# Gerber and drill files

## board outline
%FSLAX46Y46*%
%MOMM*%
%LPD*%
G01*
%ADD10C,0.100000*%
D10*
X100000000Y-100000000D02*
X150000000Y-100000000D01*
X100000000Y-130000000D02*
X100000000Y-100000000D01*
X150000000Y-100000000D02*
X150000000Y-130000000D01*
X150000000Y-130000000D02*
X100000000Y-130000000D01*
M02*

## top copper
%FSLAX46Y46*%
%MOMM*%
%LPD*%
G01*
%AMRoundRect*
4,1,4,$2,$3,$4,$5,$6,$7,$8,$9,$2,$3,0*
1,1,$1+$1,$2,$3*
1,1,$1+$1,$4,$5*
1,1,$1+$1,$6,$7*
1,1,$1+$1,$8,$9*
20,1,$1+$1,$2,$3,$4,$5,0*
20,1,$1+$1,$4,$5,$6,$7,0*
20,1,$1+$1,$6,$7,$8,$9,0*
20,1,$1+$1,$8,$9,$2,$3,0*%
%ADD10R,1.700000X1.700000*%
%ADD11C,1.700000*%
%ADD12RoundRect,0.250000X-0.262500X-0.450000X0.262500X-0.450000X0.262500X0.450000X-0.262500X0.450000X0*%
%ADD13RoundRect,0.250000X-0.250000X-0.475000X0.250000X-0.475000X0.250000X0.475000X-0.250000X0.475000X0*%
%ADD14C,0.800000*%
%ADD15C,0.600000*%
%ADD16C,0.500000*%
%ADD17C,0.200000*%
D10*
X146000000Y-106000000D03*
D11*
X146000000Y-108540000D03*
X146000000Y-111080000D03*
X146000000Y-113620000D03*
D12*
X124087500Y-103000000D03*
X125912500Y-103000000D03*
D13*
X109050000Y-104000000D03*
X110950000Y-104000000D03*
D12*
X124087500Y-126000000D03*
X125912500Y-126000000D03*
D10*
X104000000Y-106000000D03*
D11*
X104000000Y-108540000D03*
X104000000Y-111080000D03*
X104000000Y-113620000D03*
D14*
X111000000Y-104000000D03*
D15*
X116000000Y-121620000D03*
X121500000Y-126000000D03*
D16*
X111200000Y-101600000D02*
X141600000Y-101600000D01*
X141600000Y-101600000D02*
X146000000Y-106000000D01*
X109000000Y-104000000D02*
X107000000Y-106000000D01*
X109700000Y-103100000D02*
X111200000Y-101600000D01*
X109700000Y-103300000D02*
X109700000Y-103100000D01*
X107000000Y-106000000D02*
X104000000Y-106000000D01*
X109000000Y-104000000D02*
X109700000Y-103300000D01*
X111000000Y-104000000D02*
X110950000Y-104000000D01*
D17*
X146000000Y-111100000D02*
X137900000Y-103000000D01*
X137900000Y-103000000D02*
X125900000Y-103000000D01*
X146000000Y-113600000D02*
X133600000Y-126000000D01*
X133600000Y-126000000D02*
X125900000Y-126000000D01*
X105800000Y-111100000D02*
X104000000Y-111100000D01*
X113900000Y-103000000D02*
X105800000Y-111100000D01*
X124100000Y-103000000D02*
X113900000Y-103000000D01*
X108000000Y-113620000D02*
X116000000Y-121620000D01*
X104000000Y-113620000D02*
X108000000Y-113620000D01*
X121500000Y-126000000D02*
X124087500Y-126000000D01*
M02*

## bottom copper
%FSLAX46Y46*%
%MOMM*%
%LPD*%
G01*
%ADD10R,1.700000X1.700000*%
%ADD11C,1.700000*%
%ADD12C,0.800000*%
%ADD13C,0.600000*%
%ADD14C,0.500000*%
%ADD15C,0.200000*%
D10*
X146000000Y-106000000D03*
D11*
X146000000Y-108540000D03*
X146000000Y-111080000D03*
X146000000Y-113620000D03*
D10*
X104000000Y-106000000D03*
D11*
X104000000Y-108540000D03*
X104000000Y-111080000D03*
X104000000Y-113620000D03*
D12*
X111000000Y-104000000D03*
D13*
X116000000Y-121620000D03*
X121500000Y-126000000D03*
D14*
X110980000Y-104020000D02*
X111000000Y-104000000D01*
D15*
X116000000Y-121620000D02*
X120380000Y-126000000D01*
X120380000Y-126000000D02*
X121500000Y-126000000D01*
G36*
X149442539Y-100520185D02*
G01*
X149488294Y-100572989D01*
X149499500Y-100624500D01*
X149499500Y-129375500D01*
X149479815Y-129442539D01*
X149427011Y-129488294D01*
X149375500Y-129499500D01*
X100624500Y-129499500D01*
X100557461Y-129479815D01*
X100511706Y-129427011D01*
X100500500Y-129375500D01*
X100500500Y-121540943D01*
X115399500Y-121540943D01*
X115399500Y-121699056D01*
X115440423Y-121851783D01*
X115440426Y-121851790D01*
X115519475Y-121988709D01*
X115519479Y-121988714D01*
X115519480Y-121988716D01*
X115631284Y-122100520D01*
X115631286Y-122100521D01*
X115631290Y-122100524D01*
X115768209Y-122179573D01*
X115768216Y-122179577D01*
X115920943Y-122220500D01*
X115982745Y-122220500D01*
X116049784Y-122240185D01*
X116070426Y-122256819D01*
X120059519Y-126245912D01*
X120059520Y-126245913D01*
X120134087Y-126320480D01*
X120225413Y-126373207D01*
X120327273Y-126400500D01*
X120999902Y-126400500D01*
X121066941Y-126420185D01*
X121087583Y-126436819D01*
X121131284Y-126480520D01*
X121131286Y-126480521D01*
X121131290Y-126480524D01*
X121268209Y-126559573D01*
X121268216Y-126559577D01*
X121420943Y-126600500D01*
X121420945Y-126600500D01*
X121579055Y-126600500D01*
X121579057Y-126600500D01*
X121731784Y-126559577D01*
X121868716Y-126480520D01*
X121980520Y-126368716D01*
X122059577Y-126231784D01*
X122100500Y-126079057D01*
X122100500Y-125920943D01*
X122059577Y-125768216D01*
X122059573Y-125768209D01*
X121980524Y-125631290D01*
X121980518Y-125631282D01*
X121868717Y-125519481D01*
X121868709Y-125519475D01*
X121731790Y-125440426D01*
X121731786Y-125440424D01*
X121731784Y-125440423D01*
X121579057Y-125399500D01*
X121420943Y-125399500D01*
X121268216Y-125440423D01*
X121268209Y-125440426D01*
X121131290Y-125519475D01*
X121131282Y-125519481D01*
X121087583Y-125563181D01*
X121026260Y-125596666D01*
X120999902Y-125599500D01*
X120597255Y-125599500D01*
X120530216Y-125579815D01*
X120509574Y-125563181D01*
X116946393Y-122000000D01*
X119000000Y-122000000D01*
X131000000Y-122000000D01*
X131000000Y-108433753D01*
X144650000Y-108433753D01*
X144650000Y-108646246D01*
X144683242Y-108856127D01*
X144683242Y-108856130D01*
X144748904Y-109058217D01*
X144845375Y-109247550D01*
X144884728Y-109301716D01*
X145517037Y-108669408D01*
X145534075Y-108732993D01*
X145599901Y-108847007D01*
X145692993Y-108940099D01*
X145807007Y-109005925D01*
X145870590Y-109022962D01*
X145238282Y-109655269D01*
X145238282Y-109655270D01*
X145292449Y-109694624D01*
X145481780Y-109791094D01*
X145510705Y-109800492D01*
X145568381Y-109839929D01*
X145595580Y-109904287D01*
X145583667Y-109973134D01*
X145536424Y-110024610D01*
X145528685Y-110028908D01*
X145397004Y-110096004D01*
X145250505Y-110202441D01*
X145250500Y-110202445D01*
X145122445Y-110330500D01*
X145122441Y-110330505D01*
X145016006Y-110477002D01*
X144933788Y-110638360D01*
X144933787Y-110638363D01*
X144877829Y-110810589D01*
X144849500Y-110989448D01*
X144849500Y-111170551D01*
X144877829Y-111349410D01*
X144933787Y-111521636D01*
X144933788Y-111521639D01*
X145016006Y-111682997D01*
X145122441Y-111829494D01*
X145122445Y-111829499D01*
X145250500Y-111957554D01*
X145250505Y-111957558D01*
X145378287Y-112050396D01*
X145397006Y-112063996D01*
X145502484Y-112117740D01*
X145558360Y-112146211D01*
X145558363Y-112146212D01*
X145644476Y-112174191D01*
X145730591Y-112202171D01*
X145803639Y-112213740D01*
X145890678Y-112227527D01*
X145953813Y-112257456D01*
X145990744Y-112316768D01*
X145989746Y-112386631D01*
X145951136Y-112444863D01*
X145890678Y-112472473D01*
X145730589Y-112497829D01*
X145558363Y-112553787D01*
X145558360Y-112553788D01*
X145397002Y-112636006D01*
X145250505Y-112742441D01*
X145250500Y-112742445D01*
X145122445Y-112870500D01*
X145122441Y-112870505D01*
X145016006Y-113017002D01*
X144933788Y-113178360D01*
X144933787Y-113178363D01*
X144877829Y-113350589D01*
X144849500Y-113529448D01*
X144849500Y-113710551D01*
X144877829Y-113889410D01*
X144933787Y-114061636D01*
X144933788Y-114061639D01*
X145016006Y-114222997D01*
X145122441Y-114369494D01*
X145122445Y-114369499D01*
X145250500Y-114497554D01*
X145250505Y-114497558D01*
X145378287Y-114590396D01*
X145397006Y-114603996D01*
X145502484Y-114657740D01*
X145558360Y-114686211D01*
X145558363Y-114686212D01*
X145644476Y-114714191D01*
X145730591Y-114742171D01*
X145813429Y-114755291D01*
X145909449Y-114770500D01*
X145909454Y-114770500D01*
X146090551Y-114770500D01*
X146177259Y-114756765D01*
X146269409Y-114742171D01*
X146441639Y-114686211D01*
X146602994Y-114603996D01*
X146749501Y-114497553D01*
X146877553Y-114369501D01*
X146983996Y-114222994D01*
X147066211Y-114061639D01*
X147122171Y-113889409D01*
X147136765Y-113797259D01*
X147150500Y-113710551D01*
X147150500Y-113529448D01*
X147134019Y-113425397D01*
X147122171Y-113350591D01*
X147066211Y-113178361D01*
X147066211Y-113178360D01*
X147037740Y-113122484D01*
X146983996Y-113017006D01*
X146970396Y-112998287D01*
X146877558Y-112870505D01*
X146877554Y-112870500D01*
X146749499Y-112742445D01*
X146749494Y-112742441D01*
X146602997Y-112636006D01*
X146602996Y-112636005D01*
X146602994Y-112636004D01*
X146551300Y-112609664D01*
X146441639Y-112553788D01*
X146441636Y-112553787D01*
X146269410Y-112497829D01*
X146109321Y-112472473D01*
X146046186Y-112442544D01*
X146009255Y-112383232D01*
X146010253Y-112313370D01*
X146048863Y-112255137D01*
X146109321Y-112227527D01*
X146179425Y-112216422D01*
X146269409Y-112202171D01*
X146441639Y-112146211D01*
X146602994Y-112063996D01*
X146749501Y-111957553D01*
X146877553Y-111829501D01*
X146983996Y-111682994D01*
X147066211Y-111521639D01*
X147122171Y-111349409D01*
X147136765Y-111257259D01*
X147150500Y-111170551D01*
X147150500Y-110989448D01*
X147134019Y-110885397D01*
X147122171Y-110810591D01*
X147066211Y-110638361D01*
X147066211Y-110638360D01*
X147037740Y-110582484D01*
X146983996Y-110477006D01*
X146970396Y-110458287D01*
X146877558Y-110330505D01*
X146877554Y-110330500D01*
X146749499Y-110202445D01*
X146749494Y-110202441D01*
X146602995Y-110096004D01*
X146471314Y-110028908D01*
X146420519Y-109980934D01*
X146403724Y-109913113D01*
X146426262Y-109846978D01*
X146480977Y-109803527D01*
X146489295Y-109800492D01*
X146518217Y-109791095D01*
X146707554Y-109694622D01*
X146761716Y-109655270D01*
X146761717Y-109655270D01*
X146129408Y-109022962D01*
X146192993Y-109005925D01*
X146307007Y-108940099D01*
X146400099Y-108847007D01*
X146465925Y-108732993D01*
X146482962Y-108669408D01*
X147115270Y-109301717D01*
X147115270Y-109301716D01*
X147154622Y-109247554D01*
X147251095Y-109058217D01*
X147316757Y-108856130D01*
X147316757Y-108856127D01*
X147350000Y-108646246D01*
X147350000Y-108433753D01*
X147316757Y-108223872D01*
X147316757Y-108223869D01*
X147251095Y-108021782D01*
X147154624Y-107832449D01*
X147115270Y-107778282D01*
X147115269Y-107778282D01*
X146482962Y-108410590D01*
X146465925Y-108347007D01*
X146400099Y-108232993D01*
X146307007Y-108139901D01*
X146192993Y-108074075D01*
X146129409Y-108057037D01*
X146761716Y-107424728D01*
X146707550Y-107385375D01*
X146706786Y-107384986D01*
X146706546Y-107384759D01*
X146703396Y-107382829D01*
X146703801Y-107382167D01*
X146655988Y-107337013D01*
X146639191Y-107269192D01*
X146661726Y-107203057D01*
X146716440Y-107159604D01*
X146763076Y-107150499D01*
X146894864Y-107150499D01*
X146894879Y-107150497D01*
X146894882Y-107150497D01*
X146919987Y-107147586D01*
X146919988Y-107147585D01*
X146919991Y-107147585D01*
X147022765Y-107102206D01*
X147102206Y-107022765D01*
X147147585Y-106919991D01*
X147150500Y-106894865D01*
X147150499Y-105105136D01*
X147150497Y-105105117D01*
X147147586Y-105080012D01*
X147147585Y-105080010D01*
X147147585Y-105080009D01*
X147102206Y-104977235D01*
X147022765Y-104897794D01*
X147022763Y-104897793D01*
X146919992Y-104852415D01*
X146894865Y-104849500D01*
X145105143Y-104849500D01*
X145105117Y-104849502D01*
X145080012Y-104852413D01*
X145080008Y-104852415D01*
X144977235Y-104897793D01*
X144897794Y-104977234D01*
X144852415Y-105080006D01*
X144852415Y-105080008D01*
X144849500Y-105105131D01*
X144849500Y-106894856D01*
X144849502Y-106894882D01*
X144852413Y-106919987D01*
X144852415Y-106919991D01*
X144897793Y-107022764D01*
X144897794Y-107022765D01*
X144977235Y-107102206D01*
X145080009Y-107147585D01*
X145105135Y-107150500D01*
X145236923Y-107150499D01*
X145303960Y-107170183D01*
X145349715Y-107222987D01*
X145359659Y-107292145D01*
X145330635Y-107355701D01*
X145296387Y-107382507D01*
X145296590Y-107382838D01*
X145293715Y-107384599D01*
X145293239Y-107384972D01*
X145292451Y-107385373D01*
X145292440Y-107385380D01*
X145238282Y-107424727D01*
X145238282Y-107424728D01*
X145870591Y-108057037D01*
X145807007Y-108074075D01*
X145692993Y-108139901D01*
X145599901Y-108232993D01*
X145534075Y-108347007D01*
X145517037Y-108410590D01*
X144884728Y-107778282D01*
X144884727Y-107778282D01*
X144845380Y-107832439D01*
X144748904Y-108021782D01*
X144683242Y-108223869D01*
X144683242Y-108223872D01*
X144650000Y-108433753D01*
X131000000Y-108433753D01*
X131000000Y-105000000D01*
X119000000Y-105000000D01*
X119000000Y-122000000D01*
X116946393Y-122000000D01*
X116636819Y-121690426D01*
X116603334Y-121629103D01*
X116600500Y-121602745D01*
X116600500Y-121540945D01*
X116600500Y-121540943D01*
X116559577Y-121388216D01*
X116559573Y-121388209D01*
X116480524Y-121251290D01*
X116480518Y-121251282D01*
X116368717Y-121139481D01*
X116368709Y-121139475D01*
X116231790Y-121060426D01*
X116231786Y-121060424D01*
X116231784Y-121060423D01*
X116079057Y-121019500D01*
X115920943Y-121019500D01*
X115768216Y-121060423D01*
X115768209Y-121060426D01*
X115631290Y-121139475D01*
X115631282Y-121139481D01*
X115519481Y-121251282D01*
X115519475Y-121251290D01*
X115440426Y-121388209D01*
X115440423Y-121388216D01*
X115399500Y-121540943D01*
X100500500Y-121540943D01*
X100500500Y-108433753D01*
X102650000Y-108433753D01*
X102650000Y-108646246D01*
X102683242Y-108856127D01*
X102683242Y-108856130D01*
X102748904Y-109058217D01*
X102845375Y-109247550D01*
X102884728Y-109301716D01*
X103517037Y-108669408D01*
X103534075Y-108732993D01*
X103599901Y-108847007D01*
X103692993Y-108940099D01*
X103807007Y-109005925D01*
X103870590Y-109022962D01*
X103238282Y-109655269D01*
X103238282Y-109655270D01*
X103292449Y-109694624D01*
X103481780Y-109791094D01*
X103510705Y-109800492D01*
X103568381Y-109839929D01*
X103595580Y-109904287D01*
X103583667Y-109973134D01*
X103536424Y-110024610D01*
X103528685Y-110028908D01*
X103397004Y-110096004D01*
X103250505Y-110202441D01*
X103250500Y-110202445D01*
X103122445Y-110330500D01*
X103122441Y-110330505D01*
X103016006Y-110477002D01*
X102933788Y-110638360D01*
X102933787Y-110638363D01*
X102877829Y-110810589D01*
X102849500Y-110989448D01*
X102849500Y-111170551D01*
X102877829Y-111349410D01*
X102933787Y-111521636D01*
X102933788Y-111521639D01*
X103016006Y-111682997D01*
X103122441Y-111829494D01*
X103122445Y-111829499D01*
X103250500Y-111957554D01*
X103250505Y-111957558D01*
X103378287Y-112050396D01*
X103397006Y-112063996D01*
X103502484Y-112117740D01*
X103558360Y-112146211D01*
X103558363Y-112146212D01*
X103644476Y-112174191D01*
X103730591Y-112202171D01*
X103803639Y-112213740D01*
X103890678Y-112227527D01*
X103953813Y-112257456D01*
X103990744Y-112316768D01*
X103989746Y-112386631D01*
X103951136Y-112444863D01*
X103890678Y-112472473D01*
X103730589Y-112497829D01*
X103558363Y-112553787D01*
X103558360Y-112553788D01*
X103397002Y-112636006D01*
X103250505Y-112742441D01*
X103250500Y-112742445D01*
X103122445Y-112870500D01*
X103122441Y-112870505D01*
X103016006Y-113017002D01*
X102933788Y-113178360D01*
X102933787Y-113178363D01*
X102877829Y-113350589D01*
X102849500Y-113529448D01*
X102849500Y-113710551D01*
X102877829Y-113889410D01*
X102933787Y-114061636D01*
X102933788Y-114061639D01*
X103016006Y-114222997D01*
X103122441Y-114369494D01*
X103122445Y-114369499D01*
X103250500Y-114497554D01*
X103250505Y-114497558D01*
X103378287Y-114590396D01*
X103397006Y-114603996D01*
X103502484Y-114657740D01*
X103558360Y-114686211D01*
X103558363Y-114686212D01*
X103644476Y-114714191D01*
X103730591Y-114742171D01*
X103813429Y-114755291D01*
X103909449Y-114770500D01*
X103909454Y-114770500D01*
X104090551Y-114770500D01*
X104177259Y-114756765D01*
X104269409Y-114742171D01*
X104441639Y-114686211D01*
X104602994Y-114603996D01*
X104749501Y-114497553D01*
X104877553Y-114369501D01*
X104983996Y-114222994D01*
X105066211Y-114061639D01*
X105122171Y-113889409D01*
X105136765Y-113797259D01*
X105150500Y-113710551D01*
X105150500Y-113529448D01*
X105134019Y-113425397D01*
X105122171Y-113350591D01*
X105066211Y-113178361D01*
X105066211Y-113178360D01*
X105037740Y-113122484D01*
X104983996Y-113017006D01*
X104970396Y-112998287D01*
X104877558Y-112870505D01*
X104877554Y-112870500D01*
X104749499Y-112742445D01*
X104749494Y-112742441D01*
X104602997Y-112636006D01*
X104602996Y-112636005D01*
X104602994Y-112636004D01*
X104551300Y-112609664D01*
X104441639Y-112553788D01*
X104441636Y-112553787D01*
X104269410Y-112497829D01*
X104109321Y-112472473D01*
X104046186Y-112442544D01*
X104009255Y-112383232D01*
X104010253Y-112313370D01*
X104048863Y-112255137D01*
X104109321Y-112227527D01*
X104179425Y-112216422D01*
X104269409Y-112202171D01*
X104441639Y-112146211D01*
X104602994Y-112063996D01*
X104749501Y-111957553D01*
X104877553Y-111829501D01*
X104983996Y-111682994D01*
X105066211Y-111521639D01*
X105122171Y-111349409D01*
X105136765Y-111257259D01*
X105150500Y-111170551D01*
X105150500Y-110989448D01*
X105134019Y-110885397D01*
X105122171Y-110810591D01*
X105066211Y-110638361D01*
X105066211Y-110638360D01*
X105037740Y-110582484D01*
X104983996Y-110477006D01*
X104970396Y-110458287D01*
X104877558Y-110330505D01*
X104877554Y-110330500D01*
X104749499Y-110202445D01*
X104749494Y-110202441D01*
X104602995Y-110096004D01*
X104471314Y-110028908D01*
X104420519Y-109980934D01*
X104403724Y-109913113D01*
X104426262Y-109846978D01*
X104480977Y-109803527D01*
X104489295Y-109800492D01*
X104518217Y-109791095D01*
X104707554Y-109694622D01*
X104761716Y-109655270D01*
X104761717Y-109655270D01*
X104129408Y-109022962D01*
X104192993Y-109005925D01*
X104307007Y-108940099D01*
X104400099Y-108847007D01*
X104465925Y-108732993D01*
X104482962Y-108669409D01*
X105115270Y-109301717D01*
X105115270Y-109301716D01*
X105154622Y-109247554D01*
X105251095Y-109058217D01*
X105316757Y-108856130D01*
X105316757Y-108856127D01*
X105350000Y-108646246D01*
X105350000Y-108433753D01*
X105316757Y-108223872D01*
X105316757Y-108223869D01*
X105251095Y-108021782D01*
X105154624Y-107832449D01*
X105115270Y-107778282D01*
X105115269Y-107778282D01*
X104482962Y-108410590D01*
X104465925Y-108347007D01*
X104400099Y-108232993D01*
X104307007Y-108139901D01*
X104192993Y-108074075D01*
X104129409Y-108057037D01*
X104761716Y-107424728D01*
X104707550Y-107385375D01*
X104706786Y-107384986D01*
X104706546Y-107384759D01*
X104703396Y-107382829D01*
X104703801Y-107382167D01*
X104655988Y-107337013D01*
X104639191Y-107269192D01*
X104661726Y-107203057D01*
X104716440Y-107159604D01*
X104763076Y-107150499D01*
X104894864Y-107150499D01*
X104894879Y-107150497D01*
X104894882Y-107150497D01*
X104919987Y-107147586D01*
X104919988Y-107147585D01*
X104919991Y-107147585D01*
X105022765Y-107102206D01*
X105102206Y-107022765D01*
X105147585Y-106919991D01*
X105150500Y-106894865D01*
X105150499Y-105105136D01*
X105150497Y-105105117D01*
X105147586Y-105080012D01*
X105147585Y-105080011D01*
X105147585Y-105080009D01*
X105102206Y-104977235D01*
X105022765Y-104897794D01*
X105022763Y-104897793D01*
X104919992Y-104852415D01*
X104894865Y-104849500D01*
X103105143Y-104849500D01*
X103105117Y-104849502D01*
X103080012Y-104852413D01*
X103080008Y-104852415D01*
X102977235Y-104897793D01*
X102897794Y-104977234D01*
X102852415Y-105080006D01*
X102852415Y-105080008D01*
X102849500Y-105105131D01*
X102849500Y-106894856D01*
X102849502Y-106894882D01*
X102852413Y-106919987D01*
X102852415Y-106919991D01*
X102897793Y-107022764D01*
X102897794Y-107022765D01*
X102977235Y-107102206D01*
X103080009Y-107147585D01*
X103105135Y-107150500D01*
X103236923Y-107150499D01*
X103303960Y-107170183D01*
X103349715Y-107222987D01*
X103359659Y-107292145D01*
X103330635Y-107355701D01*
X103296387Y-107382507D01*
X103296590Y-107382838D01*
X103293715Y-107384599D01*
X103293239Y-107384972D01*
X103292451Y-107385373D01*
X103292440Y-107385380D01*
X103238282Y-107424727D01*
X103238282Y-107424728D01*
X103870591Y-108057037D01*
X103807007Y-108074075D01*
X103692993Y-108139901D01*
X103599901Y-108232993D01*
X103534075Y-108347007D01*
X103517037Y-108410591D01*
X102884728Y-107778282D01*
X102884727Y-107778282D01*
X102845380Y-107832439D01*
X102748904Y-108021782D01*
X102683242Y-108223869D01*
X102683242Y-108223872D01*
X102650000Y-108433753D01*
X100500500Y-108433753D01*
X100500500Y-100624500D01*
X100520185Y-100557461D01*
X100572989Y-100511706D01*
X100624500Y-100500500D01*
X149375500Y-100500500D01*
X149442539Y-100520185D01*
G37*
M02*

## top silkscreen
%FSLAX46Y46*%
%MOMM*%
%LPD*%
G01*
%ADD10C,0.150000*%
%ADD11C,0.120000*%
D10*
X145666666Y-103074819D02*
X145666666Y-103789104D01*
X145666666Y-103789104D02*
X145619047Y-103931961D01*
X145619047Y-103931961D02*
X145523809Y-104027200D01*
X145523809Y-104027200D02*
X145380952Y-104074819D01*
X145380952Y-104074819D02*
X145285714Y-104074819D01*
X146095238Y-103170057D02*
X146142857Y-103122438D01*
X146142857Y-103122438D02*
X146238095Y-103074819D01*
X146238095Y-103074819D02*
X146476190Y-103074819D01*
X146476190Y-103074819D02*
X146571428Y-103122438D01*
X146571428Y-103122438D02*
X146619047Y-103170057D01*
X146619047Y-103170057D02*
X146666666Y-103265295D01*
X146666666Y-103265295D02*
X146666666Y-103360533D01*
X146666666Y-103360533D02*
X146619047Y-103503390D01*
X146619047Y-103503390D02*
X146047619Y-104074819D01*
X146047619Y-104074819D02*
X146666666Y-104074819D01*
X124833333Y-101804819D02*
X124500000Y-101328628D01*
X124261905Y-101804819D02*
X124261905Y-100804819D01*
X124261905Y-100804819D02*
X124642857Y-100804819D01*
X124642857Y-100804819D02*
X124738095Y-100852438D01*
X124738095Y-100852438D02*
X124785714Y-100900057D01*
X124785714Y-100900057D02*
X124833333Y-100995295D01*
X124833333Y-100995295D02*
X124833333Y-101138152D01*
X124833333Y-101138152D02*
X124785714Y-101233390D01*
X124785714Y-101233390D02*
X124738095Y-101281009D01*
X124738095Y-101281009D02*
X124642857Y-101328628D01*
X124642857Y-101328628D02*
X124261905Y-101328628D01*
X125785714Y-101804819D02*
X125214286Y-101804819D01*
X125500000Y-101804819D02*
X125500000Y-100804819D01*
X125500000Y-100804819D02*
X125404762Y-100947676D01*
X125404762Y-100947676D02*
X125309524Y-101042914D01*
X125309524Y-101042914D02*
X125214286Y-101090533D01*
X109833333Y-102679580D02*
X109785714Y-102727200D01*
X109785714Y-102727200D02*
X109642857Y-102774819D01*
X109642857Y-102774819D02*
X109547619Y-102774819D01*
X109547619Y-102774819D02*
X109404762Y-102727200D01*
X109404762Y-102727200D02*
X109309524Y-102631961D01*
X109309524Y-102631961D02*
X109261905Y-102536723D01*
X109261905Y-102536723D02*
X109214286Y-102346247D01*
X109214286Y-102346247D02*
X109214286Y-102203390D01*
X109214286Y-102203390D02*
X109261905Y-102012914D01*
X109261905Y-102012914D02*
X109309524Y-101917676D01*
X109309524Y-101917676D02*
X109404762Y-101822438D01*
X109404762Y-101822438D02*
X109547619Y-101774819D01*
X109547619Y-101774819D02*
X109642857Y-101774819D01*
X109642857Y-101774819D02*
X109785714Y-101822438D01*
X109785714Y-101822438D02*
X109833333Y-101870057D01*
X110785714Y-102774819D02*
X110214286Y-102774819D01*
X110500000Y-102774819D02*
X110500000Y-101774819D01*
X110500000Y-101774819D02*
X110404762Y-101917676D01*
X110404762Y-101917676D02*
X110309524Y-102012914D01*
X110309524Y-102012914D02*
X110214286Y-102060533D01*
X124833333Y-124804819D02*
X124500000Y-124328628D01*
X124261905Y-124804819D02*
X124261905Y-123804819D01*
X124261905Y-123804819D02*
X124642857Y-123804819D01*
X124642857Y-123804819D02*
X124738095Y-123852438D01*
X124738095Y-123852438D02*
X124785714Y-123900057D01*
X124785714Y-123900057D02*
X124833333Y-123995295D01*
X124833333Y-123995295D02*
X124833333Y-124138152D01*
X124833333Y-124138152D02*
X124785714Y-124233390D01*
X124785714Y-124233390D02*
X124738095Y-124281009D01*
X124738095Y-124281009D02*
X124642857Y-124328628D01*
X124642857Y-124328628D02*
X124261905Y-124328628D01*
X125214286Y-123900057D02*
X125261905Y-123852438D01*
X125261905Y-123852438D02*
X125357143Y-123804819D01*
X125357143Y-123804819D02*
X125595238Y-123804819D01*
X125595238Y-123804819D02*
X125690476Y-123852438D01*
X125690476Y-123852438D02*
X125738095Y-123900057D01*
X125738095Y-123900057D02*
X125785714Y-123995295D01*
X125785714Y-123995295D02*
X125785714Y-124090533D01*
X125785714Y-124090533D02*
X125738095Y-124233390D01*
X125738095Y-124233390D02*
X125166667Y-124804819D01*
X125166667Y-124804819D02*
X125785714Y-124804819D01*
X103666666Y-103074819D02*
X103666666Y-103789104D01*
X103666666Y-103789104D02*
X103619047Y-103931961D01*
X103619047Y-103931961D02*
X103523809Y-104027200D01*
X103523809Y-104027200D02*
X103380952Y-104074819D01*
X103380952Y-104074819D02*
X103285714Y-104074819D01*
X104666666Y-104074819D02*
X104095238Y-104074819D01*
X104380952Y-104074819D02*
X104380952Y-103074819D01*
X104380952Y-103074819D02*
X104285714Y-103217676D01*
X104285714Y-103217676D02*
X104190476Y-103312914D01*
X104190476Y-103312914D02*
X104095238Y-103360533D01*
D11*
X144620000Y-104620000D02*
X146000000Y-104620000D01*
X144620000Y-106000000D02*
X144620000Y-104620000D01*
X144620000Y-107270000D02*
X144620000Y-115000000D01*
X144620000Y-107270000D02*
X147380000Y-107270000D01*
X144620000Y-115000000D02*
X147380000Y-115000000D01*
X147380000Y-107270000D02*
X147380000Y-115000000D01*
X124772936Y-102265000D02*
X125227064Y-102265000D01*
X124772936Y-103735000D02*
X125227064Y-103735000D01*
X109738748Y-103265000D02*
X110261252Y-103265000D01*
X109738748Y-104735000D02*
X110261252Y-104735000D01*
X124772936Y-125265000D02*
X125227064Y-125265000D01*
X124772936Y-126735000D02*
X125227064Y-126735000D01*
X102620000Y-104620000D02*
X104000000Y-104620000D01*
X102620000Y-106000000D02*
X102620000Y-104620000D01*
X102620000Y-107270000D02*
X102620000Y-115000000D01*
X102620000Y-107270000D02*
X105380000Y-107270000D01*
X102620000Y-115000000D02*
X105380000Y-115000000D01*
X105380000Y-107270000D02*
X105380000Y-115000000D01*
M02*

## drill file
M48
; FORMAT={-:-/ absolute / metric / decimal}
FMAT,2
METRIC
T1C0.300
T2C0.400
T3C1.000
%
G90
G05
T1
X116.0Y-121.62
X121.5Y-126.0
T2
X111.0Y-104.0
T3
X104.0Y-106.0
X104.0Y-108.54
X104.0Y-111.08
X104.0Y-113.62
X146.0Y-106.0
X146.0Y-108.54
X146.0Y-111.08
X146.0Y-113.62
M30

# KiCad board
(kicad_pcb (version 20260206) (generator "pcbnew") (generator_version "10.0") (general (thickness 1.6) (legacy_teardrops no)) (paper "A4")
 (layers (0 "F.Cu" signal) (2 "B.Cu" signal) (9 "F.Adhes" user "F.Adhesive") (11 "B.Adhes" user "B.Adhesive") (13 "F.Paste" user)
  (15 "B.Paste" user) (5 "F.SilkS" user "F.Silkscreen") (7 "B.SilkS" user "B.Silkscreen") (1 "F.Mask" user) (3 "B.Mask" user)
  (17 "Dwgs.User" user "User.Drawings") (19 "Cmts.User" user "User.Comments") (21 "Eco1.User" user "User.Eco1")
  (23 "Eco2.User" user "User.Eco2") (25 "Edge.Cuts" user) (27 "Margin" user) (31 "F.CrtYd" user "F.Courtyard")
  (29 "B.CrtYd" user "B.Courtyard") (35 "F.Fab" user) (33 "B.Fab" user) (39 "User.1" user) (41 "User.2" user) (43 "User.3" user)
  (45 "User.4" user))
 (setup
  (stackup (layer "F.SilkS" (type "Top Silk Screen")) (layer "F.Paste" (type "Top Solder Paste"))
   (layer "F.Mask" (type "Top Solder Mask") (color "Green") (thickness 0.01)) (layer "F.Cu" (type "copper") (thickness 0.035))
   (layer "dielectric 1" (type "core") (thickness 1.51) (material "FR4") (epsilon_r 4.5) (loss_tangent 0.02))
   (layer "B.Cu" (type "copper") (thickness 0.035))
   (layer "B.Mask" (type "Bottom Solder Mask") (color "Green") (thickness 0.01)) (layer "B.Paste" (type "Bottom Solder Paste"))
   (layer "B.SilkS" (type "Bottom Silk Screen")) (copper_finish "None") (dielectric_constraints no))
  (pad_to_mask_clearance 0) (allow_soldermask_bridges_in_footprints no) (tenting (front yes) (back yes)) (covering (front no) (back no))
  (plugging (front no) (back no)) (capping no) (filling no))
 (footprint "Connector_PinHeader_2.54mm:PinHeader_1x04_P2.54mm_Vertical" (layer "F.Cu") (at 146 106)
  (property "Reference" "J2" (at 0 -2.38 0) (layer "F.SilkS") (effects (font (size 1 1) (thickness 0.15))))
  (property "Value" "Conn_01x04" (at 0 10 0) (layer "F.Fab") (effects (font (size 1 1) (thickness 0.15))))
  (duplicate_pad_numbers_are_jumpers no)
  (fp_line (start -1.38 -1.38) (end 0 -1.38) (stroke (width 0.12) (type solid)) (layer "F.SilkS"))
  (fp_line (start -1.38 0) (end -1.38 -1.38) (stroke (width 0.12) (type solid)) (layer "F.SilkS"))
  (fp_line (start -1.38 1.27) (end -1.38 9) (stroke (width 0.12) (type solid)) (layer "F.SilkS"))
  (fp_line (start -1.38 1.27) (end 1.38 1.27) (stroke (width 0.12) (type solid)) (layer "F.SilkS"))
  (fp_line (start -1.38 9) (end 1.38 9) (stroke (width 0.12) (type solid)) (layer "F.SilkS"))
  (fp_line (start 1.38 1.27) (end 1.38 9) (stroke (width 0.12) (type solid)) (layer "F.SilkS"))
  (pad "1" thru_hole rect (at 0 0) (size 1.7 1.7) (drill 1) (layers "*.Cu" "*.Mask") (remove_unused_layers no) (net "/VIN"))
  (pad "2" thru_hole circle (at 0 2.54) (size 1.7 1.7) (drill 1) (layers "*.Cu" "*.Mask") (remove_unused_layers no) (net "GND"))
  (pad "3" thru_hole circle (at 0 5.08) (size 1.7 1.7) (drill 1) (layers "*.Cu" "*.Mask") (remove_unused_layers no) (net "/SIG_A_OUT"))
  (pad "4" thru_hole circle (at 0 7.62) (size 1.7 1.7) (drill 1) (layers "*.Cu" "*.Mask") (remove_unused_layers no) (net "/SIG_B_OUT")))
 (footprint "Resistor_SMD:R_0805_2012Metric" (layer "F.Cu") (at 125 103)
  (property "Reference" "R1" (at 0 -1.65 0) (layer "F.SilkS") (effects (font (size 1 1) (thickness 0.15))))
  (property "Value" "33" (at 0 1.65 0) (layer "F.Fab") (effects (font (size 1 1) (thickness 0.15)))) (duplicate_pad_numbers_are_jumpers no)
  (fp_line (start -0.227064 -0.735) (end 0.227064 -0.735) (stroke (width 0.12) (type solid)) (layer "F.SilkS"))
  (fp_line (start -0.227064 0.735) (end 0.227064 0.735) (stroke (width 0.12) (type solid)) (layer "F.SilkS"))
  (pad "1" smd roundrect (at -0.9125 0) (size 1.025 1.4) (layers "F.Cu" "F.Mask" "F.Paste") (roundrect_rratio 0.243902) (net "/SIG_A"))
  (pad "2" smd roundrect (at 0.9125 0) (size 1.025 1.4) (layers "F.Cu" "F.Mask" "F.Paste") (roundrect_rratio 0.243902) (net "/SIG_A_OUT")))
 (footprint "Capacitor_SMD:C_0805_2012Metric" (layer "F.Cu") (at 110 104)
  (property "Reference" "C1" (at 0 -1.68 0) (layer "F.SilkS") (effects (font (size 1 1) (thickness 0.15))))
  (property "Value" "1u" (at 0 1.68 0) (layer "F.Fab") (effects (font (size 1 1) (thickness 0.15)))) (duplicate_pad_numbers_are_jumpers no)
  (fp_line (start -0.261252 -0.735) (end 0.261252 -0.735) (stroke (width 0.12) (type solid)) (layer "F.SilkS"))
  (fp_line (start -0.261252 0.735) (end 0.261252 0.735) (stroke (width 0.12) (type solid)) (layer "F.SilkS"))
  (pad "1" smd roundrect (at -0.95 0) (size 1 1.45) (layers "F.Cu" "F.Mask" "F.Paste") (roundrect_rratio 0.25) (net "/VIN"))
  (pad "2" smd roundrect (at 0.95 0) (size 1 1.45) (layers "F.Cu" "F.Mask" "F.Paste") (roundrect_rratio 0.25) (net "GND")))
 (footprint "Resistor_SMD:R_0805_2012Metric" (layer "F.Cu") (at 125 126)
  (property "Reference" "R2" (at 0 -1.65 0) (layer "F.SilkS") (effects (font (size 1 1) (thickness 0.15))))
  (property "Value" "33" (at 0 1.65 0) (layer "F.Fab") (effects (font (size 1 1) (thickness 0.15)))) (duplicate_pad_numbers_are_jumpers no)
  (fp_line (start -0.227064 -0.735) (end 0.227064 -0.735) (stroke (width 0.12) (type solid)) (layer "F.SilkS"))
  (fp_line (start -0.227064 0.735) (end 0.227064 0.735) (stroke (width 0.12) (type solid)) (layer "F.SilkS"))
  (pad "1" smd roundrect (at -0.9125 0) (size 1.025 1.4) (layers "F.Cu" "F.Mask" "F.Paste") (roundrect_rratio 0.243902) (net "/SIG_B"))
  (pad "2" smd roundrect (at 0.9125 0) (size 1.025 1.4) (layers "F.Cu" "F.Mask" "F.Paste") (roundrect_rratio 0.243902) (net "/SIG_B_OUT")))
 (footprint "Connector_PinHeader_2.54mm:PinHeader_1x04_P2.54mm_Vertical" (layer "F.Cu") (at 104 106)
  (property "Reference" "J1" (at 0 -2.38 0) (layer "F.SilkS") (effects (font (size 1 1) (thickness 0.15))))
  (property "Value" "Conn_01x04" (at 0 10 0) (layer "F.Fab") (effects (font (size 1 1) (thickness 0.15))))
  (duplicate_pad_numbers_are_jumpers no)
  (fp_line (start -1.38 -1.38) (end 0 -1.38) (stroke (width 0.12) (type solid)) (layer "F.SilkS"))
  (fp_line (start -1.38 0) (end -1.38 -1.38) (stroke (width 0.12) (type solid)) (layer "F.SilkS"))
  (fp_line (start -1.38 1.27) (end -1.38 9) (stroke (width 0.12) (type solid)) (layer "F.SilkS"))
  (fp_line (start -1.38 1.27) (end 1.38 1.27) (stroke (width 0.12) (type solid)) (layer "F.SilkS"))
  (fp_line (start -1.38 9) (end 1.38 9) (stroke (width 0.12) (type solid)) (layer "F.SilkS"))
  (fp_line (start 1.38 1.27) (end 1.38 9) (stroke (width 0.12) (type solid)) (layer "F.SilkS"))
  (pad "1" thru_hole rect (at 0 0) (size 1.7 1.7) (drill 1) (layers "*.Cu" "*.Mask") (remove_unused_layers no) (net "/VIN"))
  (pad "2" thru_hole circle (at 0 2.54) (size 1.7 1.7) (drill 1) (layers "*.Cu" "*.Mask") (remove_unused_layers no) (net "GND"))
  (pad "3" thru_hole circle (at 0 5.08) (size 1.7 1.7) (drill 1) (layers "*.Cu" "*.Mask") (remove_unused_layers no) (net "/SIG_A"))
  (pad "4" thru_hole circle (at 0 7.62) (size 1.7 1.7) (drill 1) (layers "*.Cu" "*.Mask") (remove_unused_layers no) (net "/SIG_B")))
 (gr_line (start 100 100) (end 150 100) (stroke (width 0.1) (type default)) (layer "Edge.Cuts"))
 (gr_line (start 100 130) (end 100 100) (stroke (width 0.1) (type default)) (layer "Edge.Cuts"))
 (gr_line (start 150 100) (end 150 130) (stroke (width 0.1) (type default)) (layer "Edge.Cuts"))
 (gr_line (start 150 130) (end 100 130) (stroke (width 0.1) (type default)) (layer "Edge.Cuts"))
 (segment (start 111.2 101.6) (end 141.6 101.6) (width 0.5) (layer "F.Cu") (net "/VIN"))
 (segment (start 141.6 101.6) (end 146 106) (width 0.5) (layer "F.Cu") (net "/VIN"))
 (segment (start 109 104) (end 107 106) (width 0.5) (layer "F.Cu") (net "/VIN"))
 (segment (start 109.7 103.1) (end 111.2 101.6) (width 0.5) (layer "F.Cu") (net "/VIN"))
 (segment (start 109.7 103.3) (end 109.7 103.1) (width 0.5) (layer "F.Cu") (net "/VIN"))
 (segment (start 107 106) (end 104 106) (width 0.5) (layer "F.Cu") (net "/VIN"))
 (segment (start 109 104) (end 109.7 103.3) (width 0.5) (layer "F.Cu") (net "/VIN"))
 (segment (start 111 104) (end 110.95 104) (width 0.5) (layer "F.Cu") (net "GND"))
 (via (at 111 104) (size 0.8) (drill 0.4) (layers "F.Cu" "B.Cu") (capping yes) (filling yes) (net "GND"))
 (segment (start 110.98 104.02) (end 111 104) (width 0.5) (layer "B.Cu") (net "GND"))
 (segment (start 146 111.1) (end 137.9 103) (width 0.2) (layer "F.Cu") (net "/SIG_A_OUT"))
 (segment (start 137.9 103) (end 125.9 103) (width 0.2) (layer "F.Cu") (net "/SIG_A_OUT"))
 (segment (start 146 113.6) (end 133.6 126) (width 0.2) (layer "F.Cu") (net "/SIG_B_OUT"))
 (segment (start 133.6 126) (end 125.9 126) (width 0.2) (layer "F.Cu") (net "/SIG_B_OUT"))
 (segment (start 105.8 111.1) (end 104 111.1) (width 0.2) (layer "F.Cu") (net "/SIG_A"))
 (segment (start 113.9 103) (end 105.8 111.1) (width 0.2) (layer "F.Cu") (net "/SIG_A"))
 (segment (start 124.1 103) (end 113.9 103) (width 0.2) (layer "F.Cu") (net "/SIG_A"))
 (segment (start 108 113.62) (end 116 121.62) (width 0.2) (locked yes) (layer "F.Cu") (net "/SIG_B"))
 (segment (start 104 113.62) (end 108 113.62) (width 0.2) (locked yes) (layer "F.Cu") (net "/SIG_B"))
 (segment (start 121.5 126) (end 124.0875 126) (width 0.2) (locked yes) (layer "F.Cu") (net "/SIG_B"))
 (via (at 116 121.62) (size 0.6) (drill 0.3) (layers "F.Cu" "B.Cu") (locked yes) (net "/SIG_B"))
 (via (at 121.5 126) (size 0.6) (drill 0.3) (layers "F.Cu" "B.Cu") (locked yes) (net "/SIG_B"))
 (segment (start 116 121.62) (end 120.38 126) (width 0.2) (locked yes) (layer "B.Cu") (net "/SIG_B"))
 (segment (start 120.38 126) (end 121.5 126) (width 0.2) (locked yes) (layer "B.Cu") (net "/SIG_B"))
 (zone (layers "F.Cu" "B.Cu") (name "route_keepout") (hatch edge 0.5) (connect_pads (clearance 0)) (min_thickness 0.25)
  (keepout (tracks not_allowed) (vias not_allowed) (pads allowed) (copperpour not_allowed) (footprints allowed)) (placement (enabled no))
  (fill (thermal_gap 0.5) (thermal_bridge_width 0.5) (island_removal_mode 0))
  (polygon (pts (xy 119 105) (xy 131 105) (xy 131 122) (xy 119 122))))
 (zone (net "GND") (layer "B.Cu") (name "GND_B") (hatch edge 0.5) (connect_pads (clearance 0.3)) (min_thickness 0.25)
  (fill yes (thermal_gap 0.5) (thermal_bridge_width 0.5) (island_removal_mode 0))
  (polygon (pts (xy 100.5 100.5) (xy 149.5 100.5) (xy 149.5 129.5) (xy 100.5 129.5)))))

